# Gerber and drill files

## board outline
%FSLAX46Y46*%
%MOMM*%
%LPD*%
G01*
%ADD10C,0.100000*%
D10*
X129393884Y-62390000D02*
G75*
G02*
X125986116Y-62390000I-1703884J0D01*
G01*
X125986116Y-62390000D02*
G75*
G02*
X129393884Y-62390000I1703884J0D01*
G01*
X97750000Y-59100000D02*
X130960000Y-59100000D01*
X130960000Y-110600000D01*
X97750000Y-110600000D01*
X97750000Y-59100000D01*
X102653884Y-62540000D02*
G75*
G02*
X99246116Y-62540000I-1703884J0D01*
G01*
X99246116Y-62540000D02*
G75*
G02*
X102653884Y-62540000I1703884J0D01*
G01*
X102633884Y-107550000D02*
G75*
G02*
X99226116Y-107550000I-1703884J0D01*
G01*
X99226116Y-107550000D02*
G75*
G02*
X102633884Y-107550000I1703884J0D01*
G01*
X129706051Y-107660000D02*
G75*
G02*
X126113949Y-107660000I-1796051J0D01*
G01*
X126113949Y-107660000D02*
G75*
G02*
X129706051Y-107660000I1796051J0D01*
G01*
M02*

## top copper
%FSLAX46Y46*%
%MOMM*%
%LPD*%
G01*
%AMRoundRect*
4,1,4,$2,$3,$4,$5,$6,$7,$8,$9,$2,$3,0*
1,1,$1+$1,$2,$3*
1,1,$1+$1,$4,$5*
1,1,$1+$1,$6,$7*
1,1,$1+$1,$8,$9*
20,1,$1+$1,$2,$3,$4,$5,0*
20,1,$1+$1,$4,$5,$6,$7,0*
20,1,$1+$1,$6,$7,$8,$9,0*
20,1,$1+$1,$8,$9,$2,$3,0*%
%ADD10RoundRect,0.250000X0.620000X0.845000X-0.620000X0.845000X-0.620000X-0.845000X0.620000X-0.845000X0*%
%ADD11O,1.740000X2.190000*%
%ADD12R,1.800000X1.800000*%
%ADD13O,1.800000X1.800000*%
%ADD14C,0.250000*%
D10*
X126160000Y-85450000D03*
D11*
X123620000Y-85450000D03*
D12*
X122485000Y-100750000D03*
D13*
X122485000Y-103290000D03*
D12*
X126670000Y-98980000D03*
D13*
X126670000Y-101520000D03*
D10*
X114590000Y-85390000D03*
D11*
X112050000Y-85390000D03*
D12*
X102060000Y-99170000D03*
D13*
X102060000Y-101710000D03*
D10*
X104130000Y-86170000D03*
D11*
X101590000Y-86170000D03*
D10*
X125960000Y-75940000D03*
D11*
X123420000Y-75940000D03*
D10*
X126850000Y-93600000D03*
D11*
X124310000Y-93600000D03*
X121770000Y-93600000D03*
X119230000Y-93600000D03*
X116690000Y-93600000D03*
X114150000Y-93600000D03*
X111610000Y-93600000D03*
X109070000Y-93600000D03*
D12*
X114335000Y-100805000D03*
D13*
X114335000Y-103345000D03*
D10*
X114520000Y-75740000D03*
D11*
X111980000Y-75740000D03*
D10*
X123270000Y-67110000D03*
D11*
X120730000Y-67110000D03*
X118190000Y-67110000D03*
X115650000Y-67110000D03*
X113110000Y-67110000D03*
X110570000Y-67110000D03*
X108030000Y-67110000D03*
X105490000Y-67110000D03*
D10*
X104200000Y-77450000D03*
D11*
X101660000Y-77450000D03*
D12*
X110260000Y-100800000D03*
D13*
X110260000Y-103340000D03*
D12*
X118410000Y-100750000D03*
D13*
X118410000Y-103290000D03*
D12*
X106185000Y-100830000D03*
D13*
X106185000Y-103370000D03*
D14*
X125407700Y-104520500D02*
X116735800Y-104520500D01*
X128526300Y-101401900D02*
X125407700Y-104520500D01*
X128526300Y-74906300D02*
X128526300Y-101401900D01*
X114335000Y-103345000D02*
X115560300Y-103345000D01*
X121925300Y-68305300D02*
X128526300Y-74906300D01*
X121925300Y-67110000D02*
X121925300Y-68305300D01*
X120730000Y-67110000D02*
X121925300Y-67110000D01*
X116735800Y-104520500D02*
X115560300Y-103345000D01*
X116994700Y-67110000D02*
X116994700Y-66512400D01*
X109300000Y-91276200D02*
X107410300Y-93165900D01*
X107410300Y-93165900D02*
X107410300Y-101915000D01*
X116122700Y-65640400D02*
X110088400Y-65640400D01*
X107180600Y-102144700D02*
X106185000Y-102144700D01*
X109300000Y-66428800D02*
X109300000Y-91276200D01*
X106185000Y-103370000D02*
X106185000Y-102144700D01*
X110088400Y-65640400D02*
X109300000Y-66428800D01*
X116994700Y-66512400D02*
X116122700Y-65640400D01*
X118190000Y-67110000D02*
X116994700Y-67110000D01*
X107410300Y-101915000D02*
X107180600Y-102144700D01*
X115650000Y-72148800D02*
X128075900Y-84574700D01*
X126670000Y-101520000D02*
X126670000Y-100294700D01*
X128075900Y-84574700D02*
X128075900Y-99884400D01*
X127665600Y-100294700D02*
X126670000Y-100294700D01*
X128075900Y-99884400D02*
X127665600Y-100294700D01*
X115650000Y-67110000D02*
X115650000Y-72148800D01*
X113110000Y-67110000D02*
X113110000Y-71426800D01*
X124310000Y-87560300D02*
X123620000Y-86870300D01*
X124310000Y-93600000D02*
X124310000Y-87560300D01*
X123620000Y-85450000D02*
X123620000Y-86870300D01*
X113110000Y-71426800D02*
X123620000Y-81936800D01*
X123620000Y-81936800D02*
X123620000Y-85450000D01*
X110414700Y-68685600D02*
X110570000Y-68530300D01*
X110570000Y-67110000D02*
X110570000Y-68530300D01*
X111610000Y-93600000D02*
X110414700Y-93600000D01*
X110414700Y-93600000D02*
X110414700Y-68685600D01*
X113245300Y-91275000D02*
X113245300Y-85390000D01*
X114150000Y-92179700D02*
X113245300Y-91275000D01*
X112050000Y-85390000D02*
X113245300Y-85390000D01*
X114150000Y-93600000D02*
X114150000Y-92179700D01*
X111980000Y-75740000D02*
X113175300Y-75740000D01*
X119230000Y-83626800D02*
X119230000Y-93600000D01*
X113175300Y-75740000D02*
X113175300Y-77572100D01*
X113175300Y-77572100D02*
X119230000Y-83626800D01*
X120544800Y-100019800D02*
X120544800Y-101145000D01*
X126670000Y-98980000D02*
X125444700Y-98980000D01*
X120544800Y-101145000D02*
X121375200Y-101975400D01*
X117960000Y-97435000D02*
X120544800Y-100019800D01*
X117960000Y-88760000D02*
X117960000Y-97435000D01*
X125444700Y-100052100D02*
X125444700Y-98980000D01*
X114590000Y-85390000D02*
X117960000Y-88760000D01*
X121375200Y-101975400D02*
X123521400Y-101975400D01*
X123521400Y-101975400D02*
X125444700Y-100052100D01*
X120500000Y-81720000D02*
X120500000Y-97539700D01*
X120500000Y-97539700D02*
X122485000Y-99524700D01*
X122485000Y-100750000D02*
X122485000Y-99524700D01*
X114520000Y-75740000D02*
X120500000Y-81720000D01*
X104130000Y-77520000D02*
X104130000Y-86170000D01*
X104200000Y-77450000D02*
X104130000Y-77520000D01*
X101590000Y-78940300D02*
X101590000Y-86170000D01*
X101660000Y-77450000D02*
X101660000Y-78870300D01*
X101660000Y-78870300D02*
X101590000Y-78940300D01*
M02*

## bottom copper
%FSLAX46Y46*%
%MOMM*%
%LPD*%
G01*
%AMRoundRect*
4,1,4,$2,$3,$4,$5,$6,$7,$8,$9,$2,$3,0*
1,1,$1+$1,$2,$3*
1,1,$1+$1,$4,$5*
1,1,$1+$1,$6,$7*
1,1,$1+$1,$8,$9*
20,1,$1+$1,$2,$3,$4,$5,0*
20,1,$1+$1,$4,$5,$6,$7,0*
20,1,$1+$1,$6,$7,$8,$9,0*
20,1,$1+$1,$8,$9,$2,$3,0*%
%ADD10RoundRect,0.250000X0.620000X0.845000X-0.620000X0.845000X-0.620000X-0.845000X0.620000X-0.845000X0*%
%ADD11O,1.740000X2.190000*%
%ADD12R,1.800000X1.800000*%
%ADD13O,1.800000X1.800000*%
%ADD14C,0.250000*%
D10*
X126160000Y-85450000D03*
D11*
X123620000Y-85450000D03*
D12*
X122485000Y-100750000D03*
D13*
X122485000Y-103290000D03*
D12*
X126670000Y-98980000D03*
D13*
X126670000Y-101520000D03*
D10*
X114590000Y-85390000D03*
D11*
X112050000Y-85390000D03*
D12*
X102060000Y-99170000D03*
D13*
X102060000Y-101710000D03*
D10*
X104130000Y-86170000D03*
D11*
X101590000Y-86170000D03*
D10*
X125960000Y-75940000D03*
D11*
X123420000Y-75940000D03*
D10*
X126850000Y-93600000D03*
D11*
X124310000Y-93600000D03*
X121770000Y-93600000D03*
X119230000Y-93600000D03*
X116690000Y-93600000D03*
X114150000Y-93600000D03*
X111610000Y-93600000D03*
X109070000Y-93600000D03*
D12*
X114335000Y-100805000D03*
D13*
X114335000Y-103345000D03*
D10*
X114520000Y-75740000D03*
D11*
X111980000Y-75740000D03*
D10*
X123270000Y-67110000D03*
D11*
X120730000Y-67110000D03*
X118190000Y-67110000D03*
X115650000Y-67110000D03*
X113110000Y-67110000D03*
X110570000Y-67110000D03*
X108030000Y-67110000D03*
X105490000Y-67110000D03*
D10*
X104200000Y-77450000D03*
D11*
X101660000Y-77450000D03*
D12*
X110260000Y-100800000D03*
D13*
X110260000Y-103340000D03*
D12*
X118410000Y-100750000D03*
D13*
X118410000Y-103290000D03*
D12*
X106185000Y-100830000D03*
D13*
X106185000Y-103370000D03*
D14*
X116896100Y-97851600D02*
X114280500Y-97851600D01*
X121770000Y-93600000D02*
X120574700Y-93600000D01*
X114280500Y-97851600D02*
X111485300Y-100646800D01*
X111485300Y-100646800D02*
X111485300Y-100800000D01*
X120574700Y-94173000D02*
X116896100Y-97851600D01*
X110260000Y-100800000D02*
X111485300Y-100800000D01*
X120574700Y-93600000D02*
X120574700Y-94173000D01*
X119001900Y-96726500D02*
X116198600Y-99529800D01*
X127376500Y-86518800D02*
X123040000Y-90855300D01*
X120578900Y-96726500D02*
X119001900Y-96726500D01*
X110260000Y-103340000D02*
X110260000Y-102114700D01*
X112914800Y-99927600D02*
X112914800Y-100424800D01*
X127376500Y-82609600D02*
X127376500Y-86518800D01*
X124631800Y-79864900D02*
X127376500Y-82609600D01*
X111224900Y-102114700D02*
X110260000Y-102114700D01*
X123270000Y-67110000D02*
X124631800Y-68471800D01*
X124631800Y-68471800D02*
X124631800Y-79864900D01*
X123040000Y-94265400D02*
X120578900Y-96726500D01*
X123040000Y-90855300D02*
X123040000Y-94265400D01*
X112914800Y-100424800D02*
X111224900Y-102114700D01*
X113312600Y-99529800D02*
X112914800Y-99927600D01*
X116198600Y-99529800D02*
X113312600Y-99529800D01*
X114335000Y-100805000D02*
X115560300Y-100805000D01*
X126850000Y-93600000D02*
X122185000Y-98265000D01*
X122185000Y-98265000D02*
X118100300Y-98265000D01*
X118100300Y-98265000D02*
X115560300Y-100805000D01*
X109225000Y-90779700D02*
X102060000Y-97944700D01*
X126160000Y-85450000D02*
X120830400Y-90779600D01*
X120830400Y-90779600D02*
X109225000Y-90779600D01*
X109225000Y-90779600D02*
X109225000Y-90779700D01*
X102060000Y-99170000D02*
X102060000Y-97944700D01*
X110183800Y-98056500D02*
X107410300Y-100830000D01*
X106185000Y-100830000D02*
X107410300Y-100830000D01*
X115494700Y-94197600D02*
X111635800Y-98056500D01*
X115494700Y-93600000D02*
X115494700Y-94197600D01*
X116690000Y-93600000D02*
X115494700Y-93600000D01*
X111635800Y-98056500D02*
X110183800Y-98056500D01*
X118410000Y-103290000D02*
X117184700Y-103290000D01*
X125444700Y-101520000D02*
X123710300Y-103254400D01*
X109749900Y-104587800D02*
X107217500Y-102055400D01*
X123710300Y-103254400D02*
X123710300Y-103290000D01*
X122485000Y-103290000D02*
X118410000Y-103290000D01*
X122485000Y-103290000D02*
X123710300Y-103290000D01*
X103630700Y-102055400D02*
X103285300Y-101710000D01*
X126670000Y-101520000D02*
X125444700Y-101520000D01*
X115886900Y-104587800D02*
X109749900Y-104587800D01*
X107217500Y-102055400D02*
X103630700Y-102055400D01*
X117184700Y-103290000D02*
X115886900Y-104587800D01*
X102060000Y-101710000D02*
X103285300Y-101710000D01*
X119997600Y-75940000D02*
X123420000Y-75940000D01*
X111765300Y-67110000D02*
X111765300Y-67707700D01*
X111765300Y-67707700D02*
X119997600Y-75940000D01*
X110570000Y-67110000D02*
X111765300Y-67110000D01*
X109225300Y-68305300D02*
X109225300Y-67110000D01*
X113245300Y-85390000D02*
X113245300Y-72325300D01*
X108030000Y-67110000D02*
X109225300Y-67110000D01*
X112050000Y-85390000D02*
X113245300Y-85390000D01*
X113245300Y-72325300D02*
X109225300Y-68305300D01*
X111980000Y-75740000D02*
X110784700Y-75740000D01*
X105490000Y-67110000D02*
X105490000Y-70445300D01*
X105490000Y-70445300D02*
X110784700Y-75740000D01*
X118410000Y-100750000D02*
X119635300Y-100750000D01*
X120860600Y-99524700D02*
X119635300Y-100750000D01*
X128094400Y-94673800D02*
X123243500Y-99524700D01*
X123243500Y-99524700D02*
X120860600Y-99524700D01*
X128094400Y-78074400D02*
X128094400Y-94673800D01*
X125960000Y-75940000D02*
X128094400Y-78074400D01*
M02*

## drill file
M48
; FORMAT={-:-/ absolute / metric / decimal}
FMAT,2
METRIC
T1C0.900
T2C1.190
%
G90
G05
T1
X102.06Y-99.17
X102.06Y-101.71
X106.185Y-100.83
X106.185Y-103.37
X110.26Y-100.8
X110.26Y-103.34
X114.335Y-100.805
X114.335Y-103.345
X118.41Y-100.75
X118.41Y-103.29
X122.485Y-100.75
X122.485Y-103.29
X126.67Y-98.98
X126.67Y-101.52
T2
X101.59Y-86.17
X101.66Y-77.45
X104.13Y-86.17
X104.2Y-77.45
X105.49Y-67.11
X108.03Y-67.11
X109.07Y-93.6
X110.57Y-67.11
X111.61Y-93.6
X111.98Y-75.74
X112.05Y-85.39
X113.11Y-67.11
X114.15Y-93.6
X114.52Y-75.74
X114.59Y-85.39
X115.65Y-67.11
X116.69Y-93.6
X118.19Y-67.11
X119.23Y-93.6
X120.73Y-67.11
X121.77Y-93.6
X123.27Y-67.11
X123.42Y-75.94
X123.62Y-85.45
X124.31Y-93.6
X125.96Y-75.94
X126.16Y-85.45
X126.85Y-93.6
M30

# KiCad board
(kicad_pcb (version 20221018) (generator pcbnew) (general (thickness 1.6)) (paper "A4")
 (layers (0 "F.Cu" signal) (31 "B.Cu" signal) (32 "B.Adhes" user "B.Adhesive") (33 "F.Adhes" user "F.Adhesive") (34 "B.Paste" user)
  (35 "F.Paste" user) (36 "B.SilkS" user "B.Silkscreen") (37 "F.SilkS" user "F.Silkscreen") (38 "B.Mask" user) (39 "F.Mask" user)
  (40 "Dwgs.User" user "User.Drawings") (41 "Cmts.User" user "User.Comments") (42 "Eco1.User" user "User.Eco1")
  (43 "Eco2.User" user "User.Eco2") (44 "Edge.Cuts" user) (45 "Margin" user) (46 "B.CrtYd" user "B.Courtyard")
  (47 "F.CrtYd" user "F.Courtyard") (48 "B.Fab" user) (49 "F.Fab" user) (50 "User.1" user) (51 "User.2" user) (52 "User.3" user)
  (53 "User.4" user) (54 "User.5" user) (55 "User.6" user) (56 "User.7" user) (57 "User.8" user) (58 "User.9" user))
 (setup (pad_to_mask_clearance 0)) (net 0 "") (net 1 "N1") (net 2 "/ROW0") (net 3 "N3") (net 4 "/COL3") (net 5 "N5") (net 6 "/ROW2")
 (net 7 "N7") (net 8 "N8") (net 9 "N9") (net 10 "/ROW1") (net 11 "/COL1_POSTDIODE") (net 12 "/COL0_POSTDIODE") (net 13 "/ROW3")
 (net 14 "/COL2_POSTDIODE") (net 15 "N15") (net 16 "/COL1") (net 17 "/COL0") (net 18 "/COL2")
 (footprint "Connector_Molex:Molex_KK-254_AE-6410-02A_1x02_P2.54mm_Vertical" (layer "F.Cu") (at 126.16 85.45 180)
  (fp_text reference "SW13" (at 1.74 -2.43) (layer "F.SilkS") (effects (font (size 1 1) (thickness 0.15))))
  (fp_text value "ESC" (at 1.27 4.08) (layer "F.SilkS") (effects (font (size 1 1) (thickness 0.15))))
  (pad "1" thru_hole roundrect (at 0 0 180) (size 1.74 2.19) (drill 1.19) (layers "*.Cu" "*.Mask") (roundrect_rratio 0.1436781609)
   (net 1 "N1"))
  (pad "2" thru_hole oval (at 2.54 0 180) (size 1.74 2.19) (drill 1.19) (layers "*.Cu" "*.Mask") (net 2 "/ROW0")))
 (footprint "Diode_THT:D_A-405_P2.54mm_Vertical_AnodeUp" (layer "F.Cu") (at 122.485 100.75 -90)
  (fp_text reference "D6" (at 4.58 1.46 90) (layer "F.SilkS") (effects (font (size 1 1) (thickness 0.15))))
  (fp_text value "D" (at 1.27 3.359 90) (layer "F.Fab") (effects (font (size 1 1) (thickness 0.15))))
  (pad "1" thru_hole rect (at 0 0 270) (size 1.8 1.8) (drill 0.9) (layers "*.Cu" "*.Mask") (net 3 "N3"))
  (pad "2" thru_hole oval (at 2.54 0 270) (size 1.8 1.8) (drill 0.9) (layers "*.Cu" "*.Mask") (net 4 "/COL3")))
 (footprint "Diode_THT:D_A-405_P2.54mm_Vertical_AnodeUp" (layer "F.Cu") (at 126.67 98.98 -90)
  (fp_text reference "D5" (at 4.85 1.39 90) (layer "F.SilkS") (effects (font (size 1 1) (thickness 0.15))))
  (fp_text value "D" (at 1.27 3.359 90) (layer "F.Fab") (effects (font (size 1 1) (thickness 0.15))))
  (pad "1" thru_hole rect (at 0 0 270) (size 1.8 1.8) (drill 0.9) (layers "*.Cu" "*.Mask") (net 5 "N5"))
  (pad "2" thru_hole oval (at 2.54 0 270) (size 1.8 1.8) (drill 0.9) (layers "*.Cu" "*.Mask") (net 4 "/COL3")))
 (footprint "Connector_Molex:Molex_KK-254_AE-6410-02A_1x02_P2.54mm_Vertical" (layer "F.Cu") (at 114.59 85.39 180)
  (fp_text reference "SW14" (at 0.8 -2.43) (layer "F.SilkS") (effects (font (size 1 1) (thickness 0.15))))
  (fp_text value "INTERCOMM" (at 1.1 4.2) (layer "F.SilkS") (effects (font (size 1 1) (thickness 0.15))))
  (pad "1" thru_hole roundrect (at 0 0 180) (size 1.74 2.19) (drill 1.19) (layers "*.Cu" "*.Mask") (roundrect_rratio 0.1436781609)
   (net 5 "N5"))
  (pad "2" thru_hole oval (at 2.54 0 180) (size 1.74 2.19) (drill 1.19) (layers "*.Cu" "*.Mask") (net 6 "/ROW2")))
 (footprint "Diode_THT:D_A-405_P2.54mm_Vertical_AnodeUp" (layer "F.Cu") (at 102.06 99.17 -90)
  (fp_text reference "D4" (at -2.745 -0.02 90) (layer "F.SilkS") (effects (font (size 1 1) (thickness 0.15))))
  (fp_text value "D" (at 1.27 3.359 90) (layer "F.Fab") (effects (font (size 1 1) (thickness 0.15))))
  (pad "1" thru_hole rect (at 0 0 270) (size 1.8 1.8) (drill 0.9) (layers "*.Cu" "*.Mask") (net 1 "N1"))
  (pad "2" thru_hole oval (at 2.54 0 270) (size 1.8 1.8) (drill 0.9) (layers "*.Cu" "*.Mask") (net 4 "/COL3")))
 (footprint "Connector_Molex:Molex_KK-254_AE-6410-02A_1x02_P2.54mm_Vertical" (layer "F.Cu") (at 104.13 86.17 180)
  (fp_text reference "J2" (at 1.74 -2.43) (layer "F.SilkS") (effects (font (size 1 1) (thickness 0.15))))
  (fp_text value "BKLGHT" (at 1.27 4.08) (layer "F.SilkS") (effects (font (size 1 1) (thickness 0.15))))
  (pad "1" thru_hole roundrect (at 0 0 180) (size 1.74 2.19) (drill 1.19) (layers "*.Cu" "*.Mask") (roundrect_rratio 0.1436781609)
   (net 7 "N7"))
  (pad "2" thru_hole oval (at 2.54 0 180) (size 1.74 2.19) (drill 1.19) (layers "*.Cu" "*.Mask") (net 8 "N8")))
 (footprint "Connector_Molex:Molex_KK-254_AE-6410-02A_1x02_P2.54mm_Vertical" (layer "F.Cu") (at 125.96 75.94 180)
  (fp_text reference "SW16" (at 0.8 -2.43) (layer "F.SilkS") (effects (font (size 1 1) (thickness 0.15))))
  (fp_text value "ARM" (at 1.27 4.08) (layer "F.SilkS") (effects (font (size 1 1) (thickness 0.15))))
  (pad "1" thru_hole roundrect (at 0 0 180) (size 1.74 2.19) (drill 1.19) (layers "*.Cu" "*.Mask") (roundrect_rratio 0.1436781609)
   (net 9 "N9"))
  (pad "2" thru_hole oval (at 2.54 0 180) (size 1.74 2.19) (drill 1.19) (layers "*.Cu" "*.Mask") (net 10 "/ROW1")))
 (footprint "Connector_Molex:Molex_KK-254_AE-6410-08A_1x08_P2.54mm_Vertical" (layer "F.Cu") (at 126.85 93.6 180)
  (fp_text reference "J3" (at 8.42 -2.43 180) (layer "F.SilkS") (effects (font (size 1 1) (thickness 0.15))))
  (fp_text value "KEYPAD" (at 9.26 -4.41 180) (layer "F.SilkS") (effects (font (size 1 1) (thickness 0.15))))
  (pad "1" thru_hole roundrect (at 0 0 180) (size 1.74 2.19) (drill 1.19) (layers "*.Cu" "*.Mask") (roundrect_rratio 0.1436781609)
   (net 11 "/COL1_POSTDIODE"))
  (pad "2" thru_hole oval (at 2.54 0 180) (size 1.74 2.19) (drill 1.19) (layers "*.Cu" "*.Mask") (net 2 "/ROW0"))
  (pad "3" thru_hole oval (at 5.08 0 180) (size 1.74 2.19) (drill 1.19) (layers "*.Cu" "*.Mask") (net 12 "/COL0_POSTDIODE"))
  (pad "4" thru_hole oval (at 7.62 0 180) (size 1.74 2.19) (drill 1.19) (layers "*.Cu" "*.Mask") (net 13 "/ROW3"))
  (pad "5" thru_hole oval (at 10.16 0 180) (size 1.74 2.19) (drill 1.19) (layers "*.Cu" "*.Mask") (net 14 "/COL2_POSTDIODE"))
  (pad "6" thru_hole oval (at 12.7 0 180) (size 1.74 2.19) (drill 1.19) (layers "*.Cu" "*.Mask") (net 6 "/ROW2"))
  (pad "7" thru_hole oval (at 15.24 0 180) (size 1.74 2.19) (drill 1.19) (layers "*.Cu" "*.Mask") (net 10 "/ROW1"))
  (pad "8" thru_hole oval (at 17.78 0 180) (size 1.74 2.19) (drill 1.19) (layers "*.Cu" "*.Mask") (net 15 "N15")))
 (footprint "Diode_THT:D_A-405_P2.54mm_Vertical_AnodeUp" (layer "F.Cu") (at 114.335 100.805 -90)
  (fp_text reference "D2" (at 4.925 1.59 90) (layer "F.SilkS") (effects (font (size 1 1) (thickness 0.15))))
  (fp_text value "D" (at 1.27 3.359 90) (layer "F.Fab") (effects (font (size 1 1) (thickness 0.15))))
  (pad "1" thru_hole rect (at 0 0 270) (size 1.8 1.8) (drill 0.9) (layers "*.Cu" "*.Mask") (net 11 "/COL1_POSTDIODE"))
  (pad "2" thru_hole oval (at 2.54 0 270) (size 1.8 1.8) (drill 0.9) (layers "*.Cu" "*.Mask") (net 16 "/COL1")))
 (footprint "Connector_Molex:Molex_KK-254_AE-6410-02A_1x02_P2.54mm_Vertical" (layer "F.Cu") (at 114.52 75.74 180)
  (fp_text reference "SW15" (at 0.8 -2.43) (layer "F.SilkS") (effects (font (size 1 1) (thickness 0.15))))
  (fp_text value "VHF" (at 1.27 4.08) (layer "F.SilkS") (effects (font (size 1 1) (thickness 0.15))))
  (pad "1" thru_hole roundrect (at 0 0 180) (size 1.74 2.19) (drill 1.19) (layers "*.Cu" "*.Mask") (roundrect_rratio 0.1436781609)
   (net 3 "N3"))
  (pad "2" thru_hole oval (at 2.54 0 180) (size 1.74 2.19) (drill 1.19) (layers "*.Cu" "*.Mask") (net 13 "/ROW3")))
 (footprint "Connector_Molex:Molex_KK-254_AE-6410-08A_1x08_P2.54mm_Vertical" (layer "F.Cu") (at 123.27 67.11 180)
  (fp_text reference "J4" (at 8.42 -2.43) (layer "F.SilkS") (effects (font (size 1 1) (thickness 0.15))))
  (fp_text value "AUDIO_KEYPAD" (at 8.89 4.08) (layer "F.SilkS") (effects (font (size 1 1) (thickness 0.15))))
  (pad "1" thru_hole roundrect (at 0 0 180) (size 1.74 2.19) (drill 1.19) (layers "*.Cu" "*.Mask") (roundrect_rratio 0.1436781609)
   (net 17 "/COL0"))
  (pad "2" thru_hole oval (at 2.54 0 180) (size 1.74 2.19) (drill 1.19) (layers "*.Cu" "*.Mask") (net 16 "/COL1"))
  (pad "3" thru_hole oval (at 5.08 0 180) (size 1.74 2.19) (drill 1.19) (layers "*.Cu" "*.Mask") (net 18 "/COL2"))
  (pad "4" thru_hole oval (at 7.62 0 180) (size 1.74 2.19) (drill 1.19) (layers "*.Cu" "*.Mask") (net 4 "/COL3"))
  (pad "5" thru_hole oval (at 10.16 0 180) (size 1.74 2.19) (drill 1.19) (layers "*.Cu" "*.Mask") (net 2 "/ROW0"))
  (pad "6" thru_hole oval (at 12.7 0 180) (size 1.74 2.19) (drill 1.19) (layers "*.Cu" "*.Mask") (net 10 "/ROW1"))
  (pad "7" thru_hole oval (at 15.24 0 180) (size 1.74 2.19) (drill 1.19) (layers "*.Cu" "*.Mask") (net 6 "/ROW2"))
  (pad "8" thru_hole oval (at 17.78 0 180) (size 1.74 2.19) (drill 1.19) (layers "*.Cu" "*.Mask") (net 13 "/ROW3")))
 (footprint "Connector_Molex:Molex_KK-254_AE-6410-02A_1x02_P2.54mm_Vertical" (layer "F.Cu") (at 104.2 77.45 180)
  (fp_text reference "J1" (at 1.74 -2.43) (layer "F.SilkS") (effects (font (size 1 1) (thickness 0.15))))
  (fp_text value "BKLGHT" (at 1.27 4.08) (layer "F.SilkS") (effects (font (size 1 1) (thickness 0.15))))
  (pad "1" thru_hole roundrect (at 0 0 180) (size 1.74 2.19) (drill 1.19) (layers "*.Cu" "*.Mask") (roundrect_rratio 0.1436781609)
   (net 7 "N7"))
  (pad "2" thru_hole oval (at 2.54 0 180) (size 1.74 2.19) (drill 1.19) (layers "*.Cu" "*.Mask") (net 8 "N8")))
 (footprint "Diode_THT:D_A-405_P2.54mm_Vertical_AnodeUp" (layer "F.Cu") (at 110.26 100.8 -90)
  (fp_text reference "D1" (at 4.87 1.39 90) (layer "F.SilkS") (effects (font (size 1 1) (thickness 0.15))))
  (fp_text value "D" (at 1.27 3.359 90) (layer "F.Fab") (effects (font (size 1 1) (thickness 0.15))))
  (pad "1" thru_hole rect (at 0 0 270) (size 1.8 1.8) (drill 0.9) (layers "*.Cu" "*.Mask") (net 12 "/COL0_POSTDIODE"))
  (pad "2" thru_hole oval (at 2.54 0 270) (size 1.8 1.8) (drill 0.9) (layers "*.Cu" "*.Mask") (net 17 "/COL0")))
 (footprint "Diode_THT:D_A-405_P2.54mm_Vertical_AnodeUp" (layer "F.Cu") (at 118.41 100.75 -90)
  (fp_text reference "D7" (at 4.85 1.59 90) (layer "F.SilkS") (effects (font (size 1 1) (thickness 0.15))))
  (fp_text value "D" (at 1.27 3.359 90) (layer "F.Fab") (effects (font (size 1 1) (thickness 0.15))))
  (pad "1" thru_hole rect (at 0 0 270) (size 1.8 1.8) (drill 0.9) (layers "*.Cu" "*.Mask") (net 9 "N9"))
  (pad "2" thru_hole oval (at 2.54 0 270) (size 1.8 1.8) (drill 0.9) (layers "*.Cu" "*.Mask") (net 4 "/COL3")))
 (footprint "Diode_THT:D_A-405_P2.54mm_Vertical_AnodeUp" (layer "F.Cu") (at 106.185 100.83 -90)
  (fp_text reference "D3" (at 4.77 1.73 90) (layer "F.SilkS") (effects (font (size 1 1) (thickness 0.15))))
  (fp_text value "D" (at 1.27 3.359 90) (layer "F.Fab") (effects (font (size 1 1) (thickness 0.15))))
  (pad "1" thru_hole rect (at 0 0 270) (size 1.8 1.8) (drill 0.9) (layers "*.Cu" "*.Mask") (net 14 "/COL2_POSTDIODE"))
  (pad "2" thru_hole oval (at 2.54 0 270) (size 1.8 1.8) (drill 0.9) (layers "*.Cu" "*.Mask") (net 18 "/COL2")))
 (gr_circle locked (center 127.69 62.39) (end 128.452 60.866) (stroke (width 0.1) (type default)) (fill none) (layer "Edge.Cuts"))
 (gr_rect (start 97.75 59.1) (end 130.96 110.6) (stroke (width 0.1) (type default)) (fill none) (layer "Edge.Cuts"))
 (gr_circle locked (center 100.95 62.54) (end 101.712 61.016) (stroke (width 0.1) (type default)) (fill none) (layer "Edge.Cuts"))
 (gr_circle locked (center 100.93 107.55) (end 101.692 106.026) (stroke (width 0.1) (type default)) (fill none) (layer "Edge.Cuts"))
 (gr_circle locked (center 127.91 107.66) (end 128.164 105.882) (stroke (width 0.1) (type default)) (fill none) (layer "Edge.Cuts"))
 (segment (start 116.8961 97.8516) (end 114.2805 97.8516) (width 0.25) (layer "B.Cu") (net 12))
 (segment (start 121.77 93.6) (end 120.5747 93.6) (width 0.25) (layer "B.Cu") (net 12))
 (segment (start 114.2805 97.8516) (end 111.4853 100.6468) (width 0.25) (layer "B.Cu") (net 12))
 (segment (start 111.4853 100.6468) (end 111.4853 100.8) (width 0.25) (layer "B.Cu") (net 12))
 (segment (start 120.5747 94.173) (end 116.8961 97.8516) (width 0.25) (layer "B.Cu") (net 12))
 (segment (start 110.26 100.8) (end 111.4853 100.8) (width 0.25) (layer "B.Cu") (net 12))
 (segment (start 120.5747 93.6) (end 120.5747 94.173) (width 0.25) (layer "B.Cu") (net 12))
 (segment (start 119.0019 96.7265) (end 116.1986 99.5298) (width 0.25) (layer "B.Cu") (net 17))
 (segment (start 127.3765 86.5188) (end 123.04 90.8553) (width 0.25) (layer "B.Cu") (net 17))
 (segment (start 120.5789 96.7265) (end 119.0019 96.7265) (width 0.25) (layer "B.Cu") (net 17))
 (segment (start 110.26 103.34) (end 110.26 102.1147) (width 0.25) (layer "B.Cu") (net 17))
 (segment (start 112.9148 99.9276) (end 112.9148 100.4248) (width 0.25) (layer "B.Cu") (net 17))
 (segment (start 127.3765 82.6096) (end 127.3765 86.5188) (width 0.25) (layer "B.Cu") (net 17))
 (segment (start 124.6318 79.8649) (end 127.3765 82.6096) (width 0.25) (layer "B.Cu") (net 17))
 (segment (start 111.2249 102.1147) (end 110.26 102.1147) (width 0.25) (layer "B.Cu") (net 17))
 (segment (start 123.27 67.11) (end 124.6318 68.4718) (width 0.25) (layer "B.Cu") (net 17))
 (segment (start 124.6318 68.4718) (end 124.6318 79.8649) (width 0.25) (layer "B.Cu") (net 17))
 (segment (start 123.04 94.2654) (end 120.5789 96.7265) (width 0.25) (layer "B.Cu") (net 17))
 (segment (start 123.04 90.8553) (end 123.04 94.2654) (width 0.25) (layer "B.Cu") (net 17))
 (segment (start 112.9148 100.4248) (end 111.2249 102.1147) (width 0.25) (layer "B.Cu") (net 17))
 (segment (start 113.3126 99.5298) (end 112.9148 99.9276) (width 0.25) (layer "B.Cu") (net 17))
 (segment (start 116.1986 99.5298) (end 113.3126 99.5298) (width 0.25) (layer "B.Cu") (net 17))
 (segment (start 114.335 100.805) (end 115.5603 100.805) (width 0.25) (layer "B.Cu") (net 11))
 (segment (start 126.85 93.6) (end 122.185 98.265) (width 0.25) (layer "B.Cu") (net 11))
 (segment (start 122.185 98.265) (end 118.1003 98.265) (width 0.25) (layer "B.Cu") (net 11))
 (segment (start 118.1003 98.265) (end 115.5603 100.805) (width 0.25) (layer "B.Cu") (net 11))
 (segment (start 125.4077 104.5205) (end 116.7358 104.5205) (width 0.25) (layer "F.Cu") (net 16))
 (segment (start 128.5263 101.4019) (end 125.4077 104.5205) (width 0.25) (layer "F.Cu") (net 16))
 (segment (start 128.5263 74.9063) (end 128.5263 101.4019) (width 0.25) (layer "F.Cu") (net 16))
 (segment (start 114.335 103.345) (end 115.5603 103.345) (width 0.25) (layer "F.Cu") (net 16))
 (segment (start 121.9253 68.3053) (end 128.5263 74.9063) (width 0.25) (layer "F.Cu") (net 16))
 (segment (start 121.9253 67.11) (end 121.9253 68.3053) (width 0.25) (layer "F.Cu") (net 16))
 (segment (start 120.73 67.11) (end 121.9253 67.11) (width 0.25) (layer "F.Cu") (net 16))
 (segment (start 116.7358 104.5205) (end 115.5603 103.345) (width 0.25) (layer "F.Cu") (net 16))
 (segment (start 109.225 90.7797) (end 102.06 97.9447) (width 0.25) (layer "B.Cu") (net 1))
 (segment (start 126.16 85.45) (end 120.8304 90.7796) (width 0.25) (layer "B.Cu") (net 1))
 (segment (start 120.8304 90.7796) (end 109.225 90.7796) (width 0.25) (layer "B.Cu") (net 1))
 (segment (start 109.225 90.7796) (end 109.225 90.7797) (width 0.25) (layer "B.Cu") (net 1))
 (segment (start 102.06 99.17) (end 102.06 97.9447) (width 0.25) (layer "B.Cu") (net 1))
 (segment (start 110.1838 98.0565) (end 107.4103 100.83) (width 0.25) (layer "B.Cu") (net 14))
 (segment (start 106.185 100.83) (end 107.4103 100.83) (width 0.25) (layer "B.Cu") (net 14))
 (segment (start 115.4947 94.1976) (end 111.6358 98.0565) (width 0.25) (layer "B.Cu") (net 14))
 (segment (start 115.4947 93.6) (end 115.4947 94.1976) (width 0.25) (layer "B.Cu") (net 14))
 (segment (start 116.69 93.6) (end 115.4947 93.6) (width 0.25) (layer "B.Cu") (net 14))
 (segment (start 111.6358 98.0565) (end 110.1838 98.0565) (width 0.25) (layer "B.Cu") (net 14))
 (segment (start 116.9947 67.11) (end 116.9947 66.5124) (width 0.25) (layer "F.Cu") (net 18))
 (segment (start 109.3 91.2762) (end 107.4103 93.1659) (width 0.25) (layer "F.Cu") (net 18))
 (segment (start 107.4103 93.1659) (end 107.4103 101.915) (width 0.25) (layer "F.Cu") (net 18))
 (segment (start 116.1227 65.6404) (end 110.0884 65.6404) (width 0.25) (layer "F.Cu") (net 18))
 (segment (start 107.1806 102.1447) (end 106.185 102.1447) (width 0.25) (layer "F.Cu") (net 18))
 (segment (start 109.3 66.4288) (end 109.3 91.2762) (width 0.25) (layer "F.Cu") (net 18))
 (segment (start 106.185 103.37) (end 106.185 102.1447) (width 0.25) (layer "F.Cu") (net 18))
 (segment (start 110.0884 65.6404) (end 109.3 66.4288) (width 0.25) (layer "F.Cu") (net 18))
 (segment (start 116.9947 66.5124) (end 116.1227 65.6404) (width 0.25) (layer "F.Cu") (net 18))
 (segment (start 118.19 67.11) (end 116.9947 67.11) (width 0.25) (layer "F.Cu") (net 18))
 (segment (start 107.4103 101.915) (end 107.1806 102.1447) (width 0.25) (layer "F.Cu") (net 18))
 (segment (start 115.65 72.1488) (end 128.0759 84.5747) (width 0.25) (layer "F.Cu") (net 4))
 (segment (start 126.67 101.52) (end 126.67 100.2947) (width 0.25) (layer "F.Cu") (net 4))
 (segment (start 128.0759 84.5747) (end 128.0759 99.8844) (width 0.25) (layer "F.Cu") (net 4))
 (segment (start 127.6656 100.2947) (end 126.67 100.2947) (width 0.25) (layer "F.Cu") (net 4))
 (segment (start 128.0759 99.8844) (end 127.6656 100.2947) (width 0.25) (layer "F.Cu") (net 4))
 (segment (start 115.65 67.11) (end 115.65 72.1488) (width 0.25) (layer "F.Cu") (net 4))
 (segment (start 118.41 103.29) (end 117.1847 103.29) (width 0.25) (layer "B.Cu") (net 4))
 (segment (start 125.4447 101.52) (end 123.7103 103.2544) (width 0.25) (layer "B.Cu") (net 4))
 (segment (start 109.7499 104.5878) (end 107.2175 102.0554) (width 0.25) (layer "B.Cu") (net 4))
 (segment (start 123.7103 103.2544) (end 123.7103 103.29) (width 0.25) (layer "B.Cu") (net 4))
 (segment (start 122.485 103.29) (end 118.41 103.29) (width 0.25) (layer "B.Cu") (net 4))
 (segment (start 122.485 103.29) (end 123.7103 103.29) (width 0.25) (layer "B.Cu") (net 4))
 (segment (start 103.6307 102.0554) (end 103.2853 101.71) (width 0.25) (layer "B.Cu") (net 4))
 (segment (start 126.67 101.52) (end 125.4447 101.52) (width 0.25) (layer "B.Cu") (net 4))
 (segment (start 115.8869 104.5878) (end 109.7499 104.5878) (width 0.25) (layer "B.Cu") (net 4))
 (segment (start 107.2175 102.0554) (end 103.6307 102.0554) (width 0.25) (layer "B.Cu") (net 4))
 (segment (start 117.1847 103.29) (end 115.8869 104.5878) (width 0.25) (layer "B.Cu") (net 4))
 (segment (start 102.06 101.71) (end 103.2853 101.71) (width 0.25) (layer "B.Cu") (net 4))
 (segment (start 113.11 67.11) (end 113.11 71.4268) (width 0.25) (layer "F.Cu") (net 2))
 (segment (start 124.31 87.5603) (end 123.62 86.8703) (width 0.25) (layer "F.Cu") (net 2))
 (segment (start 124.31 93.6) (end 124.31 87.5603) (width 0.25) (layer "F.Cu") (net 2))
 (segment (start 123.62 85.45) (end 123.62 86.8703) (width 0.25) (layer "F.Cu") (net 2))
 (segment (start 113.11 71.4268) (end 123.62 81.9368) (width 0.25) (layer "F.Cu") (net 2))
 (segment (start 123.62 81.9368) (end 123.62 85.45) (width 0.25) (layer "F.Cu") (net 2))
 (segment (start 110.4147 68.6856) (end 110.57 68.5303) (width 0.25) (layer "F.Cu") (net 10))
 (segment (start 110.57 67.11) (end 110.57 68.5303) (width 0.25) (layer "F.Cu") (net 10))
 (segment (start 111.61 93.6) (end 110.4147 93.6) (width 0.25) (layer "F.Cu") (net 10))
 (segment (start 110.4147 93.6) (end 110.4147 68.6856) (width 0.25) (layer "F.Cu") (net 10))
 (segment (start 119.9976 75.94) (end 123.42 75.94) (width 0.25) (layer "B.Cu") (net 10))
 (segment (start 111.7653 67.11) (end 111.7653 67.7077) (width 0.25) (layer "B.Cu") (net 10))
 (segment (start 111.7653 67.7077) (end 119.9976 75.94) (width 0.25) (layer "B.Cu") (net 10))
 (segment (start 110.57 67.11) (end 111.7653 67.11) (width 0.25) (layer "B.Cu") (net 10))
 (segment (start 113.2453 91.275) (end 113.2453 85.39) (width 0.25) (layer "F.Cu") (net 6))
 (segment (start 114.15 92.1797) (end 113.2453 91.275) (width 0.25) (layer "F.Cu") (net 6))
 (segment (start 112.05 85.39) (end 113.2453 85.39) (width 0.25) (layer "F.Cu") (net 6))
 (segment (start 114.15 93.6) (end 114.15 92.1797) (width 0.25) (layer "F.Cu") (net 6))
 (segment (start 109.2253 68.3053) (end 109.2253 67.11) (width 0.25) (layer "B.Cu") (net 6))
 (segment (start 113.2453 85.39) (end 113.2453 72.3253) (width 0.25) (layer "B.Cu") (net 6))
 (segment (start 108.03 67.11) (end 109.2253 67.11) (width 0.25) (layer "B.Cu") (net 6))
 (segment (start 112.05 85.39) (end 113.2453 85.39) (width 0.25) (layer "B.Cu") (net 6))
 (segment (start 113.2453 72.3253) (end 109.2253 68.3053) (width 0.25) (layer "B.Cu") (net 6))
 (segment (start 111.98 75.74) (end 113.1753 75.74) (width 0.25) (layer "F.Cu") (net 13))
 (segment (start 119.23 83.6268) (end 119.23 93.6) (width 0.25) (layer "F.Cu") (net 13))
 (segment (start 113.1753 75.74) (end 113.1753 77.5721) (width 0.25) (layer "F.Cu") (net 13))
 (segment (start 113.1753 77.5721) (end 119.23 83.6268) (width 0.25) (layer "F.Cu") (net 13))
 (segment (start 111.98 75.74) (end 110.7847 75.74) (width 0.25) (layer "B.Cu") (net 13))
 (segment (start 105.49 67.11) (end 105.49 70.4453) (width 0.25) (layer "B.Cu") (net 13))
 (segment (start 105.49 70.4453) (end 110.7847 75.74) (width 0.25) (layer "B.Cu") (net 13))
 (segment (start 120.5448 100.0198) (end 120.5448 101.145) (width 0.25) (layer "F.Cu") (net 5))
 (segment (start 126.67 98.98) (end 125.4447 98.98) (width 0.25) (layer "F.Cu") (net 5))
 (segment (start 120.5448 101.145) (end 121.3752 101.9754) (width 0.25) (layer "F.Cu") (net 5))
 (segment (start 117.96 97.435) (end 120.5448 100.0198) (width 0.25) (layer "F.Cu") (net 5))
 (segment (start 117.96 88.76) (end 117.96 97.435) (width 0.25) (layer "F.Cu") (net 5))
 (segment (start 125.4447 100.0521) (end 125.4447 98.98) (width 0.25) (layer "F.Cu") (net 5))
 (segment (start 114.59 85.39) (end 117.96 88.76) (width 0.25) (layer "F.Cu") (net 5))
 (segment (start 121.3752 101.9754) (end 123.5214 101.9754) (width 0.25) (layer "F.Cu") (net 5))
 (segment (start 123.5214 101.9754) (end 125.4447 100.0521) (width 0.25) (layer "F.Cu") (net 5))
 (segment (start 120.5 81.72) (end 120.5 97.5397) (width 0.25) (layer "F.Cu") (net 3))
 (segment (start 120.5 97.5397) (end 122.485 99.5247) (width 0.25) (layer "F.Cu") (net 3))
 (segment (start 122.485 100.75) (end 122.485 99.5247) (width 0.25) (layer "F.Cu") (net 3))
 (segment (start 114.52 75.74) (end 120.5 81.72) (width 0.25) (layer "F.Cu") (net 3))
 (segment (start 118.41 100.75) (end 119.6353 100.75) (width 0.25) (layer "B.Cu") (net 9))
 (segment (start 120.8606 99.5247) (end 119.6353 100.75) (width 0.25) (layer "B.Cu") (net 9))
 (segment (start 128.0944 94.6738) (end 123.2435 99.5247) (width 0.25) (layer "B.Cu") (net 9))
 (segment (start 123.2435 99.5247) (end 120.8606 99.5247) (width 0.25) (layer "B.Cu") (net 9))
 (segment (start 128.0944 78.0744) (end 128.0944 94.6738) (width 0.25) (layer "B.Cu") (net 9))
 (segment (start 125.96 75.94) (end 128.0944 78.0744) (width 0.25) (layer "B.Cu") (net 9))
 (segment (start 104.13 77.52) (end 104.13 86.17) (width 0.25) (layer "F.Cu") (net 7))
 (segment (start 104.2 77.45) (end 104.13 77.52) (width 0.25) (layer "F.Cu") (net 7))
 (segment (start 101.59 78.9403) (end 101.59 86.17) (width 0.25) (layer "F.Cu") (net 8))
 (segment (start 101.66 77.45) (end 101.66 78.8703) (width 0.25) (layer "F.Cu") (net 8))
 (segment (start 101.66 78.8703) (end 101.59 78.9403) (width 0.25) (layer "F.Cu") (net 8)))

